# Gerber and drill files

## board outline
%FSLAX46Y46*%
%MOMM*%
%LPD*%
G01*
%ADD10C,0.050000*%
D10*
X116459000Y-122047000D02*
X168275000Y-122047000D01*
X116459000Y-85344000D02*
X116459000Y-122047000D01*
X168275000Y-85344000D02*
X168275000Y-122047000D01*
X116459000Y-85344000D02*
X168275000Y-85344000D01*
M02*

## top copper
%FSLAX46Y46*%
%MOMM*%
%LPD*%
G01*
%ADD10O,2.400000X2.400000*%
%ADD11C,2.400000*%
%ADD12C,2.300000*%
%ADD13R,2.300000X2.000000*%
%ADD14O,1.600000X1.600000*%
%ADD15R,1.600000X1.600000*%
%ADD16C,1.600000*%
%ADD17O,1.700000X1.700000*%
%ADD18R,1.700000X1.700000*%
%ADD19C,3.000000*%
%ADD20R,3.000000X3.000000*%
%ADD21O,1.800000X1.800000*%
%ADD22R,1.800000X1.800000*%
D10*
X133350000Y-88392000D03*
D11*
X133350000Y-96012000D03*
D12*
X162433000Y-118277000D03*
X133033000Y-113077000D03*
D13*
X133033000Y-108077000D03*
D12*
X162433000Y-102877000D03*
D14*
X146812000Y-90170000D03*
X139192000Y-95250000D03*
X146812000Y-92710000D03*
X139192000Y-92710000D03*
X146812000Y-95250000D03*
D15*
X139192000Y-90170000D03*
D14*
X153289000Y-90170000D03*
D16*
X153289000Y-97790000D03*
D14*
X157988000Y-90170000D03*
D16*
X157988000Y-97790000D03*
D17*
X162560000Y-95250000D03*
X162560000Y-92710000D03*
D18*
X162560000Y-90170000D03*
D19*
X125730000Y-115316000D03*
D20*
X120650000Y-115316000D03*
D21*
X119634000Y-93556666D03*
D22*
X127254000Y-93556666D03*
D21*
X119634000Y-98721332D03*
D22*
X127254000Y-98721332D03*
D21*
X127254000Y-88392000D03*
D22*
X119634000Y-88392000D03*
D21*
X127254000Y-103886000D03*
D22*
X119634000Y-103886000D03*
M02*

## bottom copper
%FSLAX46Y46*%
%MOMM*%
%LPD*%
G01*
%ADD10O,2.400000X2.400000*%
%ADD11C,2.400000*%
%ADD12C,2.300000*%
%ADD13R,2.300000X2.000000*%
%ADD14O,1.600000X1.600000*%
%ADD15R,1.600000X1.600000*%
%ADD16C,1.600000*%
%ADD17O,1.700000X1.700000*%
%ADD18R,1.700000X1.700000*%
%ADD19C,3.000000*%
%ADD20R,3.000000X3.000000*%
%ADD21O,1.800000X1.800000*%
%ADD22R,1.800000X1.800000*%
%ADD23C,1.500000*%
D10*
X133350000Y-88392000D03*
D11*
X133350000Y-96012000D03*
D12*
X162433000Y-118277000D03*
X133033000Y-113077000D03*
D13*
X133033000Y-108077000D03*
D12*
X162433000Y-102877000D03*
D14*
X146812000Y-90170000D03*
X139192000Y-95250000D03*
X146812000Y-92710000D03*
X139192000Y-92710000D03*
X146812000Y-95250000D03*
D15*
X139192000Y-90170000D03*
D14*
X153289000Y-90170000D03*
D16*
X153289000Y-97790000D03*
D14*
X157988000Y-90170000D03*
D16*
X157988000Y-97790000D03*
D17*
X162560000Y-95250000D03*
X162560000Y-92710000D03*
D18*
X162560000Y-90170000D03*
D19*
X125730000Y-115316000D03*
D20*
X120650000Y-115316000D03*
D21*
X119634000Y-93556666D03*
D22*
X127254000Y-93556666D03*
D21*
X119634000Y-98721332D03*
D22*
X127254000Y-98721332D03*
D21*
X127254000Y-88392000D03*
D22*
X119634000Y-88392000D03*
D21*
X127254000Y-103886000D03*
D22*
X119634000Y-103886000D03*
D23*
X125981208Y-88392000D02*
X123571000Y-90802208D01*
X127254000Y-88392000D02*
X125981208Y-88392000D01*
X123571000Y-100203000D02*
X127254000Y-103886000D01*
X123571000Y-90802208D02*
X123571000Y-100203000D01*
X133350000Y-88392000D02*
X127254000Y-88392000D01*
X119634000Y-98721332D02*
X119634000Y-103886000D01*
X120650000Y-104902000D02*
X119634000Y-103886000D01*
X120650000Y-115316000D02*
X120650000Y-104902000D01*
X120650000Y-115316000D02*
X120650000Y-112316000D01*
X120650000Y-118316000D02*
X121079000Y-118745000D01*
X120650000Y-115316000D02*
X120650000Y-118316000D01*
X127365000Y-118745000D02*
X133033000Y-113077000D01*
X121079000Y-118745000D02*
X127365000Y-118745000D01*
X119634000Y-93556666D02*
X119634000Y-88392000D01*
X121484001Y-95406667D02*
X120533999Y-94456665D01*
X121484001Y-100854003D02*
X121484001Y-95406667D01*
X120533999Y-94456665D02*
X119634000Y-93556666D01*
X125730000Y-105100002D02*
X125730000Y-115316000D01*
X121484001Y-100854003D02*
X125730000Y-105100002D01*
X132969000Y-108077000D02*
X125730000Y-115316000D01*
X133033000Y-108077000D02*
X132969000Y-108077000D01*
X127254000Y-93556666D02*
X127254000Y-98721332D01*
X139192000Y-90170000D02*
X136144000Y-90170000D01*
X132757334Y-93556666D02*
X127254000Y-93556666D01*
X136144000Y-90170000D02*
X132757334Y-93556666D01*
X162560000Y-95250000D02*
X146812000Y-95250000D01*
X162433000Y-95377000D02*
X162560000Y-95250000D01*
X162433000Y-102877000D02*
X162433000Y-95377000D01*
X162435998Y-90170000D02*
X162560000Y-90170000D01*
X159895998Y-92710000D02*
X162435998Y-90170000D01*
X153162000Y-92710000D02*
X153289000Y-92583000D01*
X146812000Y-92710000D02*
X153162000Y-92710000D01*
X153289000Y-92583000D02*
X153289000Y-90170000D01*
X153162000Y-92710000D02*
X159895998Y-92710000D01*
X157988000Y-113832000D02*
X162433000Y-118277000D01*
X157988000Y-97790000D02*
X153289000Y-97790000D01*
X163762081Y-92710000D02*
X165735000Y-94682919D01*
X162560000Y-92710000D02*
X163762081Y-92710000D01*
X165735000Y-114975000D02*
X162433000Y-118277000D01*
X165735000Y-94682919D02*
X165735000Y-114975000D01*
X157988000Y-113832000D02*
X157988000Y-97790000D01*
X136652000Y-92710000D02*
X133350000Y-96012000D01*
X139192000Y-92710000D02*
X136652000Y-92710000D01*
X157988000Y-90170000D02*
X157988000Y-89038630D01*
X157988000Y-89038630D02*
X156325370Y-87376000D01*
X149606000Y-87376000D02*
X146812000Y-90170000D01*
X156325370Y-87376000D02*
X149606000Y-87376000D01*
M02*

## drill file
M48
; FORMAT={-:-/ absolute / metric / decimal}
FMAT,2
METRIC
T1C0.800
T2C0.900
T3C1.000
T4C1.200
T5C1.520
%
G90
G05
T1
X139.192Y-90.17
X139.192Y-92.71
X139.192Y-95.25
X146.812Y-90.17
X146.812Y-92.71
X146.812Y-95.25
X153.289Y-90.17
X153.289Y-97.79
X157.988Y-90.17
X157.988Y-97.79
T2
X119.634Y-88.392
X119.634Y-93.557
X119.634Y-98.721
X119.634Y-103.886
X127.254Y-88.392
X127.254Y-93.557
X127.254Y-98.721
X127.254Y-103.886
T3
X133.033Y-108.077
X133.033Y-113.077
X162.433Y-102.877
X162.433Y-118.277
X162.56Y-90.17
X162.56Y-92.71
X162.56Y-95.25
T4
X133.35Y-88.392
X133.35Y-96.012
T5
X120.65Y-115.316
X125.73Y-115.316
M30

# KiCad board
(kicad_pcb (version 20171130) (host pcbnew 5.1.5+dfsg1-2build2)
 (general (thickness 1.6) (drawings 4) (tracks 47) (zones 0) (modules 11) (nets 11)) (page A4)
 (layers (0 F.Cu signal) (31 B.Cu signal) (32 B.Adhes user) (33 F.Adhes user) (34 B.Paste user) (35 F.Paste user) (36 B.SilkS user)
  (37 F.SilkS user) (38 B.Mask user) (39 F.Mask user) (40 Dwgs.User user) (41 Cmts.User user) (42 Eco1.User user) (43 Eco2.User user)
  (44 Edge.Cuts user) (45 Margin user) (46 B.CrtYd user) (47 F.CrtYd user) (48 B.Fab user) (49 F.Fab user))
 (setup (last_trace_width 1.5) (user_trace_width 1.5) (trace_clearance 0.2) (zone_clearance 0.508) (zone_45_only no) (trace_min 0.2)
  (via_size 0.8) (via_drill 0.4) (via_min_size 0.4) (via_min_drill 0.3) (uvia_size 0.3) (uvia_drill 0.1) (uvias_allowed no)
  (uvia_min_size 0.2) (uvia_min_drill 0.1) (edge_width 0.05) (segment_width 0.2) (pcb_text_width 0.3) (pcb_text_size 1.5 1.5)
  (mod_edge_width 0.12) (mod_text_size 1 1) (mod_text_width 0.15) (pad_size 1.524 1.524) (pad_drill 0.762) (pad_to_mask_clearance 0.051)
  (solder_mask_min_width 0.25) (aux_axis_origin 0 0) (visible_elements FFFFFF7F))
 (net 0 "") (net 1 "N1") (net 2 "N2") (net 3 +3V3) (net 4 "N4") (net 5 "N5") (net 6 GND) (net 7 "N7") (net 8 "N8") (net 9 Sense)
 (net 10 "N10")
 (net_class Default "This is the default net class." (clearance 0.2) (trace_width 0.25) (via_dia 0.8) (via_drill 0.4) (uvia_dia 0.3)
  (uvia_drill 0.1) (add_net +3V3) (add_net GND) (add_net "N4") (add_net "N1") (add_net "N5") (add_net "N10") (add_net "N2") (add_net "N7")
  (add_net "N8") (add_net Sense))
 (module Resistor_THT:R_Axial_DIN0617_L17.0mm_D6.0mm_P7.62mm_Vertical (layer F.Cu) (at 133.35 96.012 90)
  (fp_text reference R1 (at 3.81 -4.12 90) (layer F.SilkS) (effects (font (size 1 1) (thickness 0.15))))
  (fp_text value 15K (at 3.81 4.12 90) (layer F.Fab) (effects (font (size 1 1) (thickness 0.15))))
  (pad 2 thru_hole oval (at 7.62 0 90) (size 2.4 2.4) (drill 1.2) (layers *.Cu *.Mask) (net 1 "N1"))
  (pad 1 thru_hole circle (at 0 0 90) (size 2.4 2.4) (drill 1.2) (layers *.Cu *.Mask) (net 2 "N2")))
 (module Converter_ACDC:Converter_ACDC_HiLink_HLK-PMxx (layer F.Cu) (at 133.033 108.077)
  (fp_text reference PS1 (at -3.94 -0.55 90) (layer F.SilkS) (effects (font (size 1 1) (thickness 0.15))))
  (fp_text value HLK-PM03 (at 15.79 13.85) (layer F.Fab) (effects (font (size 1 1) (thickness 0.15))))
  (pad 4 thru_hole circle (at 29.4 10.2) (size 2.3 2.3) (drill 1) (layers *.Cu *.Mask) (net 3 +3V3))
  (pad 2 thru_hole circle (at 0 5) (size 2.3 2.3) (drill 1) (layers *.Cu *.Mask) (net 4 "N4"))
  (pad 1 thru_hole rect (at 0 0) (size 2.3 2) (drill 1) (layers *.Cu *.Mask) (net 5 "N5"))
  (pad 3 thru_hole circle (at 29.4 -5.2) (size 2.3 2.3) (drill 1) (layers *.Cu *.Mask) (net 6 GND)))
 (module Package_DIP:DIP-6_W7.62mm (layer F.Cu) (at 139.192 90.17)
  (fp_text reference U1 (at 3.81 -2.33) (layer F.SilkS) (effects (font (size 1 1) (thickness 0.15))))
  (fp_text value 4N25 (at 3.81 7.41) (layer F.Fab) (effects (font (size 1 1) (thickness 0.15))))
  (pad 6 thru_hole oval (at 7.62 0) (size 1.6 1.6) (drill 0.8) (layers *.Cu *.Mask) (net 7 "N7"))
  (pad 3 thru_hole oval (at 0 5.08) (size 1.6 1.6) (drill 0.8) (layers *.Cu *.Mask) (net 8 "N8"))
  (pad 5 thru_hole oval (at 7.62 2.54) (size 1.6 1.6) (drill 0.8) (layers *.Cu *.Mask) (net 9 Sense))
  (pad 2 thru_hole oval (at 0 2.54) (size 1.6 1.6) (drill 0.8) (layers *.Cu *.Mask) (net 2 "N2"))
  (pad 4 thru_hole oval (at 7.62 5.08) (size 1.6 1.6) (drill 0.8) (layers *.Cu *.Mask) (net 6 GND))
  (pad 1 thru_hole rect (at 0 0) (size 1.6 1.6) (drill 0.8) (layers *.Cu *.Mask) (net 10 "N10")))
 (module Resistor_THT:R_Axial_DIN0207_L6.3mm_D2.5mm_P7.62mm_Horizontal (layer F.Cu) (at 153.289 97.79 90)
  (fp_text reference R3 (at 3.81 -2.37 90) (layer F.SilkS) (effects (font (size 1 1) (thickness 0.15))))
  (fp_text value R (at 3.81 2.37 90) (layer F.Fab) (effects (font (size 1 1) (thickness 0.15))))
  (pad 2 thru_hole oval (at 7.62 0 90) (size 1.6 1.6) (drill 0.8) (layers *.Cu *.Mask) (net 9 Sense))
  (pad 1 thru_hole circle (at 0 0 90) (size 1.6 1.6) (drill 0.8) (layers *.Cu *.Mask) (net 3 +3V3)))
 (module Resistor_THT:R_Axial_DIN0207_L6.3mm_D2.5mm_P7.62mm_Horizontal (layer F.Cu) (at 157.988 97.79 90)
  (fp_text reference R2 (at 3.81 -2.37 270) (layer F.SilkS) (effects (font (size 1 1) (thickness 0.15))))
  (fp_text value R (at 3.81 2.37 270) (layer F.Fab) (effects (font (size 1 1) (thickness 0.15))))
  (pad 2 thru_hole oval (at 7.62 0 90) (size 1.6 1.6) (drill 0.8) (layers *.Cu *.Mask) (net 7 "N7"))
  (pad 1 thru_hole circle (at 0 0 90) (size 1.6 1.6) (drill 0.8) (layers *.Cu *.Mask) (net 3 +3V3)))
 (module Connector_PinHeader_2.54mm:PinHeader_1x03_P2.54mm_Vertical (layer F.Cu) (at 162.56 90.17)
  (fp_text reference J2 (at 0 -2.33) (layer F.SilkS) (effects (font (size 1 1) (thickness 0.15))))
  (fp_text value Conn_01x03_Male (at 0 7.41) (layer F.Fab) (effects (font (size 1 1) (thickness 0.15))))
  (pad 3 thru_hole oval (at 0 5.08) (size 1.7 1.7) (drill 1) (layers *.Cu *.Mask) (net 6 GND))
  (pad 2 thru_hole oval (at 0 2.54) (size 1.7 1.7) (drill 1) (layers *.Cu *.Mask) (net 3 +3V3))
  (pad 1 thru_hole rect (at 0 0) (size 1.7 1.7) (drill 1) (layers *.Cu *.Mask) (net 9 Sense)))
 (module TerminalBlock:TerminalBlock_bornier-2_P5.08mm (layer F.Cu) (at 120.65 115.316)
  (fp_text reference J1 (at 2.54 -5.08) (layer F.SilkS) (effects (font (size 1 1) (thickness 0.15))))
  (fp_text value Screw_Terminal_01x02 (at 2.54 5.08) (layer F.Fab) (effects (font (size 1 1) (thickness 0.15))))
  (pad 2 thru_hole circle (at 5.08 0) (size 3 3) (drill 1.52) (layers *.Cu *.Mask) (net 5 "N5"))
  (pad 1 thru_hole rect (at 0 0) (size 3 3) (drill 1.52) (layers *.Cu *.Mask) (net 4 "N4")))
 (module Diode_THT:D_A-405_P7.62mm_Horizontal (layer F.Cu) (at 127.254 93.556666 180)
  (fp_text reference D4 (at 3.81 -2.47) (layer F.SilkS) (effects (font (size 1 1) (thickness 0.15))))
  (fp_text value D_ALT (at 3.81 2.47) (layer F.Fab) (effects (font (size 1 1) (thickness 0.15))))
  (pad 2 thru_hole oval (at 7.62 0 180) (size 1.8 1.8) (drill 0.9) (layers *.Cu *.Mask) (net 5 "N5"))
  (pad 1 thru_hole rect (at 0 0 180) (size 1.8 1.8) (drill 0.9) (layers *.Cu *.Mask) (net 10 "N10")))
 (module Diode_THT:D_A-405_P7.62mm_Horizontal (layer F.Cu) (at 127.254 98.721332 180)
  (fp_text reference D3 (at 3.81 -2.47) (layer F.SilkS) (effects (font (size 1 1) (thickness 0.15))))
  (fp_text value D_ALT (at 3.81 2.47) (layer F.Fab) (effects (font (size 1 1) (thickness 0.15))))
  (pad 2 thru_hole oval (at 7.62 0 180) (size 1.8 1.8) (drill 0.9) (layers *.Cu *.Mask) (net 4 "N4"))
  (pad 1 thru_hole rect (at 0 0 180) (size 1.8 1.8) (drill 0.9) (layers *.Cu *.Mask) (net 10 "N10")))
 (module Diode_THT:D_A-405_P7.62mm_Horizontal (layer F.Cu) (at 119.634 88.392)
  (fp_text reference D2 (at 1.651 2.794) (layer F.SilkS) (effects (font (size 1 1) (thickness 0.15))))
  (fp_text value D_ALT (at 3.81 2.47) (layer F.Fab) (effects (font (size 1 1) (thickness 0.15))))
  (pad 2 thru_hole oval (at 7.62 0) (size 1.8 1.8) (drill 0.9) (layers *.Cu *.Mask) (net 1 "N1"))
  (pad 1 thru_hole rect (at 0 0) (size 1.8 1.8) (drill 0.9) (layers *.Cu *.Mask) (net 5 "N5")))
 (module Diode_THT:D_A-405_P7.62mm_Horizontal (layer F.Cu) (at 119.634 103.886)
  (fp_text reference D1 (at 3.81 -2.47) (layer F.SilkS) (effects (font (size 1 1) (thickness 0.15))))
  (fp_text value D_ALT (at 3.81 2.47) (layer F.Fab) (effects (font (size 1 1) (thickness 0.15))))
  (pad 2 thru_hole oval (at 7.62 0) (size 1.8 1.8) (drill 0.9) (layers *.Cu *.Mask) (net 1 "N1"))
  (pad 1 thru_hole rect (at 0 0) (size 1.8 1.8) (drill 0.9) (layers *.Cu *.Mask) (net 4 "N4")))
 (gr_line (start 116.459 122.047) (end 168.275 122.047) (layer Edge.Cuts) (width 0.05))
 (gr_line (start 116.459 85.344) (end 116.459 122.047) (layer Edge.Cuts) (width 0.05))
 (gr_line (start 168.275 85.344) (end 168.275 122.047) (layer Edge.Cuts) (width 0.05))
 (gr_line (start 116.459 85.344) (end 168.275 85.344) (layer Edge.Cuts) (width 0.05))
 (segment (start 125.981208 88.392) (end 123.571 90.802208) (width 1.5) (layer B.Cu) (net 1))
 (segment (start 127.254 88.392) (end 125.981208 88.392) (width 1.5) (layer B.Cu) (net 1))
 (segment (start 123.571 100.203) (end 127.254 103.886) (width 1.5) (layer B.Cu) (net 1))
 (segment (start 123.571 90.802208) (end 123.571 100.203) (width 1.5) (layer B.Cu) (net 1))
 (segment (start 133.35 88.392) (end 127.254 88.392) (width 1.5) (layer B.Cu) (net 1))
 (segment (start 119.634 98.721332) (end 119.634 103.886) (width 1.5) (layer B.Cu) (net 4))
 (segment (start 120.65 104.902) (end 119.634 103.886) (width 1.5) (layer B.Cu) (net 4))
 (segment (start 120.65 115.316) (end 120.65 104.902) (width 1.5) (layer B.Cu) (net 4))
 (segment (start 120.65 115.316) (end 120.65 112.316) (width 1.5) (layer B.Cu) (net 4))
 (segment (start 120.65 118.316) (end 121.079 118.745) (width 1.5) (layer B.Cu) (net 4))
 (segment (start 120.65 115.316) (end 120.65 118.316) (width 1.5) (layer B.Cu) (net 4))
 (segment (start 127.365 118.745) (end 133.033 113.077) (width 1.5) (layer B.Cu) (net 4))
 (segment (start 121.079 118.745) (end 127.365 118.745) (width 1.5) (layer B.Cu) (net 4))
 (segment (start 119.634 93.556666) (end 119.634 88.392) (width 1.5) (layer B.Cu) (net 5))
 (segment (start 121.484001 95.406667) (end 120.533999 94.456665) (width 1.5) (layer B.Cu) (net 5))
 (segment (start 121.484001 100.854003) (end 121.484001 95.406667) (width 1.5) (layer B.Cu) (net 5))
 (segment (start 120.533999 94.456665) (end 119.634 93.556666) (width 1.5) (layer B.Cu) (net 5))
 (segment (start 125.73 105.100002) (end 125.73 115.316) (width 1.5) (layer B.Cu) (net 5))
 (segment (start 121.484001 100.854003) (end 125.73 105.100002) (width 1.5) (layer B.Cu) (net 5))
 (segment (start 132.969 108.077) (end 125.73 115.316) (width 1.5) (layer B.Cu) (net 5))
 (segment (start 133.033 108.077) (end 132.969 108.077) (width 1.5) (layer B.Cu) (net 5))
 (segment (start 127.254 93.556666) (end 127.254 98.721332) (width 1.5) (layer B.Cu) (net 10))
 (segment (start 139.192 90.17) (end 136.144 90.17) (width 1.5) (layer B.Cu) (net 10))
 (segment (start 132.757334 93.556666) (end 127.254 93.556666) (width 1.5) (layer B.Cu) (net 10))
 (segment (start 136.144 90.17) (end 132.757334 93.556666) (width 1.5) (layer B.Cu) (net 10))
 (segment (start 162.56 95.25) (end 146.812 95.25) (width 1.5) (layer B.Cu) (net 6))
 (segment (start 162.433 95.377) (end 162.56 95.25) (width 1.5) (layer B.Cu) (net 6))
 (segment (start 162.433 102.877) (end 162.433 95.377) (width 1.5) (layer B.Cu) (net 6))
 (segment (start 162.435998 90.17) (end 162.56 90.17) (width 1.5) (layer B.Cu) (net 9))
 (segment (start 159.895998 92.71) (end 162.435998 90.17) (width 1.5) (layer B.Cu) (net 9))
 (segment (start 153.162 92.71) (end 153.289 92.583) (width 1.5) (layer B.Cu) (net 9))
 (segment (start 146.812 92.71) (end 153.162 92.71) (width 1.5) (layer B.Cu) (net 9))
 (segment (start 153.289 92.583) (end 153.289 90.17) (width 1.5) (layer B.Cu) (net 9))
 (segment (start 153.162 92.71) (end 159.895998 92.71) (width 1.5) (layer B.Cu) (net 9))
 (segment (start 157.988 113.832) (end 162.433 118.277) (width 1.5) (layer B.Cu) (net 3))
 (segment (start 157.988 97.79) (end 153.289 97.79) (width 1.5) (layer B.Cu) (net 3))
 (segment (start 163.762081 92.71) (end 165.735 94.682919) (width 1.5) (layer B.Cu) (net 3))
 (segment (start 162.56 92.71) (end 163.762081 92.71) (width 1.5) (layer B.Cu) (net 3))
 (segment (start 165.735 114.975) (end 162.433 118.277) (width 1.5) (layer B.Cu) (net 3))
 (segment (start 165.735 94.682919) (end 165.735 114.975) (width 1.5) (layer B.Cu) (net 3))
 (segment (start 157.988 113.832) (end 157.988 97.79) (width 1.5) (layer B.Cu) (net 3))
 (segment (start 136.652 92.71) (end 133.35 96.012) (width 1.5) (layer B.Cu) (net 2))
 (segment (start 139.192 92.71) (end 136.652 92.71) (width 1.5) (layer B.Cu) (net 2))
 (segment (start 157.988 90.17) (end 157.988 89.03863) (width 1.5) (layer B.Cu) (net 7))
 (segment (start 157.988 89.03863) (end 156.32537 87.376) (width 1.5) (layer B.Cu) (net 7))
 (segment (start 149.606 87.376) (end 146.812 90.17) (width 1.5) (layer B.Cu) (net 7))
 (segment (start 156.32537 87.376) (end 149.606 87.376) (width 1.5) (layer B.Cu) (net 7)))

